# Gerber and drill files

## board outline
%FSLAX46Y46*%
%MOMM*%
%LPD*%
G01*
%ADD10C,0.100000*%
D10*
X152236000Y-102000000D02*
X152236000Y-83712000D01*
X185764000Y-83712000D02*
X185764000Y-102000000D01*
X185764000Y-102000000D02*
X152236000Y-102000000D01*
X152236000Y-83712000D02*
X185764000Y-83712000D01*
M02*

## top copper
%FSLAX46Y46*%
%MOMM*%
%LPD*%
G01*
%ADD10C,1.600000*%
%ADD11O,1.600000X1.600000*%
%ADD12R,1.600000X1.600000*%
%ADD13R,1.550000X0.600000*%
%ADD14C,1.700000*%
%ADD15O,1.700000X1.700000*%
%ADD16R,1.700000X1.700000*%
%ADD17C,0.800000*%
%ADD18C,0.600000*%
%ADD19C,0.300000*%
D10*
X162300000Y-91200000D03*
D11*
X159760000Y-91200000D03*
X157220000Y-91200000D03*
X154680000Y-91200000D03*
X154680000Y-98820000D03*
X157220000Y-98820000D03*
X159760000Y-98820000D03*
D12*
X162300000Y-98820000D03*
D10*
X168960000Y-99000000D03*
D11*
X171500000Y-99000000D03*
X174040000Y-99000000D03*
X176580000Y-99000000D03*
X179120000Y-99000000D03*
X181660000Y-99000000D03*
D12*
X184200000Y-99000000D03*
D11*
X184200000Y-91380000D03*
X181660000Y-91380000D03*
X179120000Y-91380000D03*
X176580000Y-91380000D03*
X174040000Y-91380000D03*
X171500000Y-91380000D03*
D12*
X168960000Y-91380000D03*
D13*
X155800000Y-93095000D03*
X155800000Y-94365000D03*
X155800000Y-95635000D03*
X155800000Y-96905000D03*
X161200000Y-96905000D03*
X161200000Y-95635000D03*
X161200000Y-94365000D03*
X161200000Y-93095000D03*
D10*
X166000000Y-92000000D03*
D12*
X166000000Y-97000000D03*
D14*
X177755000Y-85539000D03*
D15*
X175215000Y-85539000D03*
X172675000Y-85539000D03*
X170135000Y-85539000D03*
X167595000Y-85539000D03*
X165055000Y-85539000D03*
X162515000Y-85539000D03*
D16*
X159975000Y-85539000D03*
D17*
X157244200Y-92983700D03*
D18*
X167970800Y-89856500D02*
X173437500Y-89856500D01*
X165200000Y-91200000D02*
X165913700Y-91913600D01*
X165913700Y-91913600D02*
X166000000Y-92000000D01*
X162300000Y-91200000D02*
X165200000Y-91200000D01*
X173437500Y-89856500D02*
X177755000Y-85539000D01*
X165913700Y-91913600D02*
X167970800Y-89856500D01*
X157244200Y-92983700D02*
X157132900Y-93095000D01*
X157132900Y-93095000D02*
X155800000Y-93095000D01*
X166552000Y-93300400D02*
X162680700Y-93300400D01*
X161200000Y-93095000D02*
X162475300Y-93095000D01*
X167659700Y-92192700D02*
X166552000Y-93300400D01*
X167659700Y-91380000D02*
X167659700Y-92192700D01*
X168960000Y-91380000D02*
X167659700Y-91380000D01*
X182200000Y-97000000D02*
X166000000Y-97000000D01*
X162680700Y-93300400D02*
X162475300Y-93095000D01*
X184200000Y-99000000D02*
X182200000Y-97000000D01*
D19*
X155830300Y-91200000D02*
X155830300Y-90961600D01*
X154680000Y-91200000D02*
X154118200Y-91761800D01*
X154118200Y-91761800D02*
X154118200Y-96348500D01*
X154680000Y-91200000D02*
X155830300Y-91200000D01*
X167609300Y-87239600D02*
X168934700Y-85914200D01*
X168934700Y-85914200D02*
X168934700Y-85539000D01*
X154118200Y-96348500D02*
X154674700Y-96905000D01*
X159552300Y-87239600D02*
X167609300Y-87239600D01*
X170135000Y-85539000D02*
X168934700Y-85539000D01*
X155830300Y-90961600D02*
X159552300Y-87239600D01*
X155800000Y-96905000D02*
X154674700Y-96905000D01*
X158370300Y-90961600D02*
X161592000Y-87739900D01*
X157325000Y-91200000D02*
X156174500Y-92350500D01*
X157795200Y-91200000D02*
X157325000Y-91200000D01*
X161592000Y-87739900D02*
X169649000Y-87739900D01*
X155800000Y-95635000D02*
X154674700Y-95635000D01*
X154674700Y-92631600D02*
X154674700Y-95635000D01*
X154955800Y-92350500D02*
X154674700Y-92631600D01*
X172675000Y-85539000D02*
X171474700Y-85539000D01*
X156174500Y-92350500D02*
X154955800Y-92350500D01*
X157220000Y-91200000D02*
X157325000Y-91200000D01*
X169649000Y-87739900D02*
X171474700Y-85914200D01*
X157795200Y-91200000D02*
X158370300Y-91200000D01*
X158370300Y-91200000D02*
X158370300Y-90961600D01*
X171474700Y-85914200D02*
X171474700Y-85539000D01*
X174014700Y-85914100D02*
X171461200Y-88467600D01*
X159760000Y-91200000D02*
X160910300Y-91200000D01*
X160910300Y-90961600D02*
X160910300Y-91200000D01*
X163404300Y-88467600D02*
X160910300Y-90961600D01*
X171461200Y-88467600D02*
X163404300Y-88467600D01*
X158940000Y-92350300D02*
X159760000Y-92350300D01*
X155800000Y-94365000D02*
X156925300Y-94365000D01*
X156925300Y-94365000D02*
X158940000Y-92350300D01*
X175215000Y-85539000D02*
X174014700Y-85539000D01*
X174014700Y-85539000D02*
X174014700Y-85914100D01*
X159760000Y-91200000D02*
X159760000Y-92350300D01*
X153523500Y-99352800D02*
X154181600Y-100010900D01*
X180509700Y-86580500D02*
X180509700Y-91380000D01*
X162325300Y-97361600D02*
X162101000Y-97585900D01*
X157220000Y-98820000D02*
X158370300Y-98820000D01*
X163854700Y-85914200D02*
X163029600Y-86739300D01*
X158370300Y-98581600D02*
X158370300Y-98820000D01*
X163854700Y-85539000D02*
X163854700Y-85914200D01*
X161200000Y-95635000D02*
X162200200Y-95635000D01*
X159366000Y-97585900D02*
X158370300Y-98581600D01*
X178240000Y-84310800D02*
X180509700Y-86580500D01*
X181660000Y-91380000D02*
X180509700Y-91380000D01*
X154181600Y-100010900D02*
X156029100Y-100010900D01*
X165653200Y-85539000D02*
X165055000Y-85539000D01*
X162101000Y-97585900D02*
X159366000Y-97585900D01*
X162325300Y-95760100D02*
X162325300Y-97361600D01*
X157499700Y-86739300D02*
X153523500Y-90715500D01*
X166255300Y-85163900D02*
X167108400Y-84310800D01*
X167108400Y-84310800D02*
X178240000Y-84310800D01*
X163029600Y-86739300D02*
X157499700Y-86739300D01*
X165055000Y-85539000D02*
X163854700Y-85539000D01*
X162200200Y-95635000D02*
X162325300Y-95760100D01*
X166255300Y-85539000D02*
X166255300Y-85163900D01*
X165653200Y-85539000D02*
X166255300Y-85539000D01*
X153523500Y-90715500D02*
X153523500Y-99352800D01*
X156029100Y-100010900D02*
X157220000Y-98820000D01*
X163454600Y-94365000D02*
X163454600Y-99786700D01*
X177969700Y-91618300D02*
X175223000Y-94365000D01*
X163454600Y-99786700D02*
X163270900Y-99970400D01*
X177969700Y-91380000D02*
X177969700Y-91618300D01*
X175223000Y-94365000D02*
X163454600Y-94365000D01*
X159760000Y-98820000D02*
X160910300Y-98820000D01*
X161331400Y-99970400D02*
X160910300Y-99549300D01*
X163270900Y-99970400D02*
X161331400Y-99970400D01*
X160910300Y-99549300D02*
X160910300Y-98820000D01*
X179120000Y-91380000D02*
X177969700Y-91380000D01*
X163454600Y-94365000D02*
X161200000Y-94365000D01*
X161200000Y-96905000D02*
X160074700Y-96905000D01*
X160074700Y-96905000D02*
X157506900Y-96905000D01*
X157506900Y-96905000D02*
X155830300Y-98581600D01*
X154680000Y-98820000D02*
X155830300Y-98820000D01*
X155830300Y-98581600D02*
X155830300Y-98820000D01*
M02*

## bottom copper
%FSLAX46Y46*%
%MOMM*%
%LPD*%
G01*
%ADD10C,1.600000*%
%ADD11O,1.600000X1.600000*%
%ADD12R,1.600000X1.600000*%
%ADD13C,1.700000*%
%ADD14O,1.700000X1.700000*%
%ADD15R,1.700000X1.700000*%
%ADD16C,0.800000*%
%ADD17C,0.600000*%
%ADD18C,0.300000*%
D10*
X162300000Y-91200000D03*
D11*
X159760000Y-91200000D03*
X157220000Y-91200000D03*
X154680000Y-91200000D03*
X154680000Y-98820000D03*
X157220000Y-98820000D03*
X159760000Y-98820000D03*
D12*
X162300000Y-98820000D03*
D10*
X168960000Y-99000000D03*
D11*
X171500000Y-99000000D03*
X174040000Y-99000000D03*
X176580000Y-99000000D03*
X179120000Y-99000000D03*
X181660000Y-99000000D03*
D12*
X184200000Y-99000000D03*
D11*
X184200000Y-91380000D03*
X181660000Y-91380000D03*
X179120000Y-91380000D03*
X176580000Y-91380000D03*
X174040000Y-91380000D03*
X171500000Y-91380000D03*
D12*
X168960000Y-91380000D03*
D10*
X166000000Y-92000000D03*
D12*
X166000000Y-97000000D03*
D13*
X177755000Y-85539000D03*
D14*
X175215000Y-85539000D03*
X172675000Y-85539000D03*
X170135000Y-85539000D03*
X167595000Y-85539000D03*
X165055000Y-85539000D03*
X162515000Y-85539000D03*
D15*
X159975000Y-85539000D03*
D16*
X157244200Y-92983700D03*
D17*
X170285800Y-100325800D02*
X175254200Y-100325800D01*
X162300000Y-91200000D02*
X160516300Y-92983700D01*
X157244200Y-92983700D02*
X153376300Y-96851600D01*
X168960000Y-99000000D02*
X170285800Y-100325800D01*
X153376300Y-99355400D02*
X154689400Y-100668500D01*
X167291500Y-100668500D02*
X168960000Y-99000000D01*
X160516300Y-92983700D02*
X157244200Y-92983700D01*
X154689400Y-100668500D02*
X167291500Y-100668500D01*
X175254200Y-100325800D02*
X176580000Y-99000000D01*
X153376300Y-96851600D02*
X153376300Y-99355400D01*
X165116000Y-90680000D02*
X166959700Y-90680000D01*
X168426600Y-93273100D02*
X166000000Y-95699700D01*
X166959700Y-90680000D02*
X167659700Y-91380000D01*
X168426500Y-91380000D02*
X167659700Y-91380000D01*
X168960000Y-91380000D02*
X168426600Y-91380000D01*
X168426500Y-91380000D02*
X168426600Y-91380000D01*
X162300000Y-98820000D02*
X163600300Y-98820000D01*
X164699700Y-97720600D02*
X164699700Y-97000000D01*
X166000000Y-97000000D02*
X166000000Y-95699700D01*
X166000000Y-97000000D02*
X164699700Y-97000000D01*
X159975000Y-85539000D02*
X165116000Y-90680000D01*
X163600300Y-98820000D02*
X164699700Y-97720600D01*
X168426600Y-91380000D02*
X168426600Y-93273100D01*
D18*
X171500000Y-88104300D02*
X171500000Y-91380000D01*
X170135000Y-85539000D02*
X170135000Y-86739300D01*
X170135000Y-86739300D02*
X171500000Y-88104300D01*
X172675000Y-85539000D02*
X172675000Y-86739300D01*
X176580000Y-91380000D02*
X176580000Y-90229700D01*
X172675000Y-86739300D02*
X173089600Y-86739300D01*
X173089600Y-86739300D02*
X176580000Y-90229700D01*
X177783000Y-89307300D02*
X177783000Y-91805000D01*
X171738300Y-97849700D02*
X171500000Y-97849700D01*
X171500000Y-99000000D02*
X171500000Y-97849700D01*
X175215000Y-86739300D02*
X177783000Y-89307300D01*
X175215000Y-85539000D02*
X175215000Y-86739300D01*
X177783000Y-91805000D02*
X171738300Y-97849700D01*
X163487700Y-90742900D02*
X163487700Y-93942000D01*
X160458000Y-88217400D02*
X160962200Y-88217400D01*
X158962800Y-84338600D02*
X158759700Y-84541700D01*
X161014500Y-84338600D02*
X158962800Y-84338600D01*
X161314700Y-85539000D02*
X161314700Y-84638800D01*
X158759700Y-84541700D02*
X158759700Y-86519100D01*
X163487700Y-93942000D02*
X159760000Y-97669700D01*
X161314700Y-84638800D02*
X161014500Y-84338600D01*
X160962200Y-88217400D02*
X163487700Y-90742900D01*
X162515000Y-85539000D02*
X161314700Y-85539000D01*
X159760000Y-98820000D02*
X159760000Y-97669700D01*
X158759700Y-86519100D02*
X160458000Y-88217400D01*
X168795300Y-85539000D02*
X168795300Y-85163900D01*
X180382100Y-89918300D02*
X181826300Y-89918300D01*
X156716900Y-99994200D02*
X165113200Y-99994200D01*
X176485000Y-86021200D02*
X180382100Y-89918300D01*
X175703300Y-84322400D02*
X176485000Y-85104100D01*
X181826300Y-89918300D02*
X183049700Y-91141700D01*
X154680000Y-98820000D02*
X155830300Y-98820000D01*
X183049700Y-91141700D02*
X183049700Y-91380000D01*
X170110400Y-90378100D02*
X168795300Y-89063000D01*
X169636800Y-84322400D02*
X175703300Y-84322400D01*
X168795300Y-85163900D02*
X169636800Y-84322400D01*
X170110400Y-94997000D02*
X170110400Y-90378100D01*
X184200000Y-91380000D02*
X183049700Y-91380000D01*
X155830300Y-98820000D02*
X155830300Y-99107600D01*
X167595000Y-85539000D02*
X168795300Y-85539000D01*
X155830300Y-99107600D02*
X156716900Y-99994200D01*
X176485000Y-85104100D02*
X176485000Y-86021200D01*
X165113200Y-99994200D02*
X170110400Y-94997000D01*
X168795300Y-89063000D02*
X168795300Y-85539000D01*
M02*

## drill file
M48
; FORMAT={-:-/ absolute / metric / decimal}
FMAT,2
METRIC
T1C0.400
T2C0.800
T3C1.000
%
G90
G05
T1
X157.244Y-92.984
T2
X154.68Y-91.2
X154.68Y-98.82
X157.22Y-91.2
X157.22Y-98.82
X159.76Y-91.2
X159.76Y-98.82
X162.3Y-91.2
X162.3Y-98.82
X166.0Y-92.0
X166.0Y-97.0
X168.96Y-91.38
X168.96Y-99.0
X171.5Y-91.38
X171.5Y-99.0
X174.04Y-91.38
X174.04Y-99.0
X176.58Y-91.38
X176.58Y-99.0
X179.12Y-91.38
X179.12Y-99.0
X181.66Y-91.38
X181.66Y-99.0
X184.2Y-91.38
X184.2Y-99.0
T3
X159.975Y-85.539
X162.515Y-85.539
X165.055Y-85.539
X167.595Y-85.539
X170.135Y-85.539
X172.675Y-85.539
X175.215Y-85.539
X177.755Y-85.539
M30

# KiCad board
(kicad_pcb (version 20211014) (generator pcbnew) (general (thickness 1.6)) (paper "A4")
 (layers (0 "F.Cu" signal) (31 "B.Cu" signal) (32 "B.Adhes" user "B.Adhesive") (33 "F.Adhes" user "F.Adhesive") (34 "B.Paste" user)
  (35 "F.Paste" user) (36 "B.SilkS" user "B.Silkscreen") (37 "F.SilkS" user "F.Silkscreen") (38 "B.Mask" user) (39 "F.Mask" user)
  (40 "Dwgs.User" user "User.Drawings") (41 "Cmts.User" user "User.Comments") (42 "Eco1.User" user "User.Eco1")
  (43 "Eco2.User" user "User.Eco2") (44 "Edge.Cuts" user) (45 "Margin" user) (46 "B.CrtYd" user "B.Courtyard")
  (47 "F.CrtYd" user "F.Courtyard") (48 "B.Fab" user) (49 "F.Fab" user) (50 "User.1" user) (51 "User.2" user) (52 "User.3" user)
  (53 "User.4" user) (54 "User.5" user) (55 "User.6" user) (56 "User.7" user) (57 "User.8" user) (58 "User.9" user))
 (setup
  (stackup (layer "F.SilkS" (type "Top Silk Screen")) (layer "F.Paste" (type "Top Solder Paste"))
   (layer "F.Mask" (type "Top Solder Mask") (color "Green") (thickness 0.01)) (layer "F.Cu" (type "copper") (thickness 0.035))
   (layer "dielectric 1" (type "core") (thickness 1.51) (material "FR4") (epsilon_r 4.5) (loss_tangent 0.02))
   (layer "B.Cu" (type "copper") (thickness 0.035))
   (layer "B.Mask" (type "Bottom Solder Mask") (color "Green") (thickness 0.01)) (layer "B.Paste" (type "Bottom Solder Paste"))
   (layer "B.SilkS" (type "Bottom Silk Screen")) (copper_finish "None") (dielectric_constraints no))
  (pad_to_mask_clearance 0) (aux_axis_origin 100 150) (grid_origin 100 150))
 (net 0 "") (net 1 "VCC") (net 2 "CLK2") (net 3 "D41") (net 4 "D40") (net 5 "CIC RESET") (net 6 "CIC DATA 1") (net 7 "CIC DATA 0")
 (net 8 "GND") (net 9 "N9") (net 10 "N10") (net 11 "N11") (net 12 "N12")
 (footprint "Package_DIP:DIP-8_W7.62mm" (layer "F.Cu") (at 162.3 91.2 -90)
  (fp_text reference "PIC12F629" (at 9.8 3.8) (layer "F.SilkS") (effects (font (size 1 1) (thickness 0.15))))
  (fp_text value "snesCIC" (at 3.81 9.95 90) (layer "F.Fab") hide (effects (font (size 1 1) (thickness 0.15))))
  (pad "1" thru_hole circle (at 0 0 270) (size 1.6 1.6) (drill 0.8) (layers *.Cu *.Mask) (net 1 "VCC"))
  (pad "2" thru_hole oval (at 0 2.54 270) (size 1.6 1.6) (drill 0.8) (layers *.Cu *.Mask) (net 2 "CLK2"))
  (pad "3" thru_hole oval (at 0 5.08 270) (size 1.6 1.6) (drill 0.8) (layers *.Cu *.Mask) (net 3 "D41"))
  (pad "4" thru_hole oval (at 0 7.62 270) (size 1.6 1.6) (drill 0.8) (layers *.Cu *.Mask) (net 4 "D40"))
  (pad "5" thru_hole oval (at 7.62 7.62 270) (size 1.6 1.6) (drill 0.8) (layers *.Cu *.Mask) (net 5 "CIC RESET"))
  (pad "6" thru_hole oval (at 7.62 5.08 270) (size 1.6 1.6) (drill 0.8) (layers *.Cu *.Mask) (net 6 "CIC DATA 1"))
  (pad "7" thru_hole oval (at 7.62 2.54 270) (size 1.6 1.6) (drill 0.8) (layers *.Cu *.Mask) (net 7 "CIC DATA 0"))
  (pad "8" thru_hole rect (at 7.62 0 270) (size 1.6 1.6) (drill 0.8) (layers *.Cu *.Mask) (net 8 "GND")))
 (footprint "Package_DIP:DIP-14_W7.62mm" (layer "F.Cu") (at 168.96 99 90)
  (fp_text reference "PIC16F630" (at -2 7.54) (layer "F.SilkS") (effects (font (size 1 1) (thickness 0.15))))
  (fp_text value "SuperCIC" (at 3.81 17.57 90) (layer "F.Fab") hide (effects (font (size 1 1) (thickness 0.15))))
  (pad "1" thru_hole circle (at 0 0 90) (size 1.6 1.6) (drill 0.8) (layers *.Cu *.Mask) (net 1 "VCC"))
  (pad "2" thru_hole oval (at 0 2.54 90) (size 1.6 1.6) (drill 0.8) (layers *.Cu *.Mask) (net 2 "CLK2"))
  (pad "3" thru_hole oval (at 0 5.08 90) (size 1.6 1.6) (drill 0.8) (layers *.Cu *.Mask) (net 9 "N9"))
  (pad "4" thru_hole oval (at 0 7.62 90) (size 1.6 1.6) (drill 0.8) (layers *.Cu *.Mask) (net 1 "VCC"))
  (pad "5" thru_hole oval (at 0 10.16 90) (size 1.6 1.6) (drill 0.8) (layers *.Cu *.Mask) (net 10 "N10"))
  (pad "6" thru_hole oval (at 0 12.7 90) (size 1.6 1.6) (drill 0.8) (layers *.Cu *.Mask) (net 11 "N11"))
  (pad "7" thru_hole rect (at 0 15.24 90) (size 1.6 1.6) (drill 0.8) (layers *.Cu *.Mask) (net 8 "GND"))
  (pad "8" thru_hole oval (at 7.62 15.24 90) (size 1.6 1.6) (drill 0.8) (layers *.Cu *.Mask) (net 5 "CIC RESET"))
  (pad "9" thru_hole oval (at 7.62 12.7 90) (size 1.6 1.6) (drill 0.8) (layers *.Cu *.Mask) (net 6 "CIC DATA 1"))
  (pad "10" thru_hole oval (at 7.62 10.16 90) (size 1.6 1.6) (drill 0.8) (layers *.Cu *.Mask) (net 7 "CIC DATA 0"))
  (pad "11" thru_hole oval (at 7.62 7.62 90) (size 1.6 1.6) (drill 0.8) (layers *.Cu *.Mask) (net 3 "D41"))
  (pad "12" thru_hole oval (at 7.62 5.08 90) (size 1.6 1.6) (drill 0.8) (layers *.Cu *.Mask) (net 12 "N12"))
  (pad "13" thru_hole oval (at 7.62 2.54 90) (size 1.6 1.6) (drill 0.8) (layers *.Cu *.Mask) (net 4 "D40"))
  (pad "14" thru_hole rect (at 7.62 0 90) (size 1.6 1.6) (drill 0.8) (layers *.Cu *.Mask) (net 8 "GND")))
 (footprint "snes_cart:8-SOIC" (layer "F.Cu") (at 158.5 95 90)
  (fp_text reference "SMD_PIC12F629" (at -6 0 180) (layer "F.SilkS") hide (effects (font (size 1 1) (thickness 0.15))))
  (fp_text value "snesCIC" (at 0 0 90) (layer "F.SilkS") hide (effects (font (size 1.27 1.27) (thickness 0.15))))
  (pad "1" smd rect (at 1.905 -2.7 180) (size 1.55 0.6) (layers "F.Cu" "F.Paste" "F.Mask") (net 1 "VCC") (solder_mask_margin 0.1016))
  (pad "2" smd rect (at 0.635 -2.7 180) (size 1.55 0.6) (layers "F.Cu" "F.Paste" "F.Mask") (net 2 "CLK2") (solder_mask_margin 0.1016))
  (pad "3" smd rect (at -0.635 -2.7 180) (size 1.55 0.6) (layers "F.Cu" "F.Paste" "F.Mask") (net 3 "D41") (solder_mask_margin 0.1016))
  (pad "4" smd rect (at -1.905 -2.7 180) (size 1.55 0.6) (layers "F.Cu" "F.Paste" "F.Mask") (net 4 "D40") (solder_mask_margin 0.1016))
  (pad "5" smd rect (at -1.905 2.7 180) (size 1.55 0.6) (layers "F.Cu" "F.Paste" "F.Mask") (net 5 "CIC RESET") (solder_mask_margin 0.1016))
  (pad "6" smd rect (at -0.635 2.7 180) (size 1.55 0.6) (layers "F.Cu" "F.Paste" "F.Mask") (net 6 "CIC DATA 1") (solder_mask_margin 0.1016))
  (pad "7" smd rect (at 0.635 2.7 180) (size 1.55 0.6) (layers "F.Cu" "F.Paste" "F.Mask") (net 7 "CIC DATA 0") (solder_mask_margin 0.1016))
  (pad "8" smd rect (at 1.905 2.7 180) (size 1.55 0.6) (layers "F.Cu" "F.Paste" "F.Mask") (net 8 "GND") (solder_mask_margin 0.1016)))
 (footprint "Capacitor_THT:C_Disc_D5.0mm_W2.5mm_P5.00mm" (layer "F.Cu") (at 166 92 -90)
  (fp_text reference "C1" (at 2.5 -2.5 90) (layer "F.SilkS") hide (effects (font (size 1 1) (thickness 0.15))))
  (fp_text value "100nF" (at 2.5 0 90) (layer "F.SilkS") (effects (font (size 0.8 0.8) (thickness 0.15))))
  (pad "1" thru_hole circle (at 0 0 270) (size 1.6 1.6) (drill 0.8) (layers *.Cu *.Mask) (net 1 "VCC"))
  (pad "2" thru_hole rect (at 5 0 270) (size 1.6 1.6) (drill 0.8) (layers *.Cu *.Mask) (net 8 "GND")))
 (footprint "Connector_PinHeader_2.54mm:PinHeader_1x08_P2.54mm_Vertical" (layer "B.Cu") (at 177.755 85.539 90)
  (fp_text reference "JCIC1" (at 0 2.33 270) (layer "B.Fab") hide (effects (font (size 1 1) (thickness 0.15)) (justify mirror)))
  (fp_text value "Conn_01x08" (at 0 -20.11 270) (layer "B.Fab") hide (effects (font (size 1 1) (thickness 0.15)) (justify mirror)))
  (pad "1" thru_hole circle (at 0 0 90) (size 1.7 1.7) (drill 1) (layers *.Cu *.Mask) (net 1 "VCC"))
  (pad "2" thru_hole oval (at 0 -2.54 90) (size 1.7 1.7) (drill 1) (layers *.Cu *.Mask) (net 2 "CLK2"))
  (pad "3" thru_hole oval (at 0 -5.08 90) (size 1.7 1.7) (drill 1) (layers *.Cu *.Mask) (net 3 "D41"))
  (pad "4" thru_hole oval (at 0 -7.62 90) (size 1.7 1.7) (drill 1) (layers *.Cu *.Mask) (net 4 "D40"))
  (pad "5" thru_hole oval (at 0 -10.16 90) (size 1.7 1.7) (drill 1) (layers *.Cu *.Mask) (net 5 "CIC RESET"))
  (pad "6" thru_hole oval (at 0 -12.7 90) (size 1.7 1.7) (drill 1) (layers *.Cu *.Mask) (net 6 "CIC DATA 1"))
  (pad "7" thru_hole oval (at 0 -15.24 90) (size 1.7 1.7) (drill 1) (layers *.Cu *.Mask) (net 7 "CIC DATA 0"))
  (pad "8" thru_hole rect (at 0 -17.78 90) (size 1.7 1.7) (drill 1) (layers *.Cu *.Mask) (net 8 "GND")))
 (gr_line (start 152.236 102) (end 152.236 83.712) (layer "Edge.Cuts") (width 0.1))
 (gr_line (start 185.764 83.712) (end 185.764 102) (layer "Edge.Cuts") (width 0.1))
 (gr_line (start 185.764 102) (end 152.236 102) (layer "Edge.Cuts") (width 0.1))
 (gr_line (start 152.236 83.712) (end 185.764 83.712) (layer "Edge.Cuts") (width 0.1))
 (segment (start 167.9708 89.8565) (end 173.4375 89.8565) (width 0.6) (layer "F.Cu") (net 1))
 (segment (start 165.2 91.2) (end 165.9137 91.9136) (width 0.6) (layer "F.Cu") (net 1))
 (segment (start 165.9137 91.9136) (end 166 92) (width 0.6) (layer "F.Cu") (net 1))
 (segment (start 162.3 91.2) (end 165.2 91.2) (width 0.6) (layer "F.Cu") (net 1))
 (segment (start 173.4375 89.8565) (end 177.755 85.539) (width 0.6) (layer "F.Cu") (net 1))
 (segment (start 165.9137 91.9136) (end 167.9708 89.8565) (width 0.6) (layer "F.Cu") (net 1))
 (segment (start 157.2442 92.9837) (end 157.1329 93.095) (width 0.6) (layer "F.Cu") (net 1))
 (segment (start 157.1329 93.095) (end 155.8 93.095) (width 0.6) (layer "F.Cu") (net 1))
 (via (at 157.2442 92.9837) (size 0.8) (drill 0.4) (layers "F.Cu" "B.Cu") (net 1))
 (segment (start 170.2858 100.3258) (end 175.2542 100.3258) (width 0.6) (layer "B.Cu") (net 1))
 (segment (start 162.3 91.2) (end 160.5163 92.9837) (width 0.6) (layer "B.Cu") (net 1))
 (segment (start 157.2442 92.9837) (end 153.3763 96.8516) (width 0.6) (layer "B.Cu") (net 1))
 (segment (start 168.96 99) (end 170.2858 100.3258) (width 0.6) (layer "B.Cu") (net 1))
 (segment (start 153.3763 99.3554) (end 154.6894 100.6685) (width 0.6) (layer "B.Cu") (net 1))
 (segment (start 167.2915 100.6685) (end 168.96 99) (width 0.6) (layer "B.Cu") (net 1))
 (segment (start 160.5163 92.9837) (end 157.2442 92.9837) (width 0.6) (layer "B.Cu") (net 1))
 (segment (start 154.6894 100.6685) (end 167.2915 100.6685) (width 0.6) (layer "B.Cu") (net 1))
 (segment (start 175.2542 100.3258) (end 176.58 99) (width 0.6) (layer "B.Cu") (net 1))
 (segment (start 153.3763 96.8516) (end 153.3763 99.3554) (width 0.6) (layer "B.Cu") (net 1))
 (segment (start 166.552 93.3004) (end 162.6807 93.3004) (width 0.6) (layer "F.Cu") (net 8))
 (segment (start 161.2 93.095) (end 162.4753 93.095) (width 0.6) (layer "F.Cu") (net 8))
 (segment (start 167.6597 92.1927) (end 166.552 93.3004) (width 0.6) (layer "F.Cu") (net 8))
 (segment (start 167.6597 91.38) (end 167.6597 92.1927) (width 0.6) (layer "F.Cu") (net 8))
 (segment (start 168.96 91.38) (end 167.6597 91.38) (width 0.6) (layer "F.Cu") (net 8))
 (segment (start 182.2 97) (end 166 97) (width 0.6) (layer "F.Cu") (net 8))
 (segment (start 162.6807 93.3004) (end 162.4753 93.095) (width 0.6) (layer "F.Cu") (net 8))
 (segment (start 184.2 99) (end 182.2 97) (width 0.6) (layer "F.Cu") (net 8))
 (segment (start 165.116 90.68) (end 166.9597 90.68) (width 0.6) (layer "B.Cu") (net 8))
 (segment (start 168.4266 93.2731) (end 166 95.6997) (width 0.6) (layer "B.Cu") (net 8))
 (segment (start 166.9597 90.68) (end 167.6597 91.38) (width 0.6) (layer "B.Cu") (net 8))
 (segment (start 168.4265 91.38) (end 167.6597 91.38) (width 0.6) (layer "B.Cu") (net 8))
 (segment (start 168.96 91.38) (end 168.4266 91.38) (width 0.6) (layer "B.Cu") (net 8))
 (segment (start 168.4265 91.38) (end 168.4266 91.38) (width 0.6) (layer "B.Cu") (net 8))
 (segment (start 162.3 98.82) (end 163.6003 98.82) (width 0.6) (layer "B.Cu") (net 8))
 (segment (start 164.6997 97.7206) (end 164.6997 97) (width 0.6) (layer "B.Cu") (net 8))
 (segment (start 166 97) (end 166 95.6997) (width 0.6) (layer "B.Cu") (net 8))
 (segment (start 166 97) (end 164.6997 97) (width 0.6) (layer "B.Cu") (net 8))
 (segment (start 159.975 85.539) (end 165.116 90.68) (width 0.6) (layer "B.Cu") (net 8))
 (segment (start 163.6003 98.82) (end 164.6997 97.7206) (width 0.6) (layer "B.Cu") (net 8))
 (segment (start 168.4266 91.38) (end 168.4266 93.2731) (width 0.6) (layer "B.Cu") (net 8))
 (segment (start 155.8303 91.2) (end 155.8303 90.9616) (width 0.3) (layer "F.Cu") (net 4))
 (segment (start 154.68 91.2) (end 154.1182 91.7618) (width 0.3) (layer "F.Cu") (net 4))
 (segment (start 154.1182 91.7618) (end 154.1182 96.3485) (width 0.3) (layer "F.Cu") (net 4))
 (segment (start 154.68 91.2) (end 155.8303 91.2) (width 0.3) (layer "F.Cu") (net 4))
 (segment (start 167.6093 87.2396) (end 168.9347 85.9142) (width 0.3) (layer "F.Cu") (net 4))
 (segment (start 168.9347 85.9142) (end 168.9347 85.539) (width 0.3) (layer "F.Cu") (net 4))
 (segment (start 154.1182 96.3485) (end 154.6747 96.905) (width 0.3) (layer "F.Cu") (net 4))
 (segment (start 159.5523 87.2396) (end 167.6093 87.2396) (width 0.3) (layer "F.Cu") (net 4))
 (segment (start 170.135 85.539) (end 168.9347 85.539) (width 0.3) (layer "F.Cu") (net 4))
 (segment (start 155.8303 90.9616) (end 159.5523 87.2396) (width 0.3) (layer "F.Cu") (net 4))
 (segment (start 155.8 96.905) (end 154.6747 96.905) (width 0.3) (layer "F.Cu") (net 4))
 (segment (start 171.5 88.1043) (end 171.5 91.38) (width 0.3) (layer "B.Cu") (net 4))
 (segment (start 170.135 85.539) (end 170.135 86.7393) (width 0.3) (layer "B.Cu") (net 4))
 (segment (start 170.135 86.7393) (end 171.5 88.1043) (width 0.3) (layer "B.Cu") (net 4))
 (segment (start 158.3703 90.9616) (end 161.592 87.7399) (width 0.3) (layer "F.Cu") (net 3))
 (segment (start 157.325 91.2) (end 156.1745 92.3505) (width 0.3) (layer "F.Cu") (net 3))
 (segment (start 157.7952 91.2) (end 157.325 91.2) (width 0.3) (layer "F.Cu") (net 3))
 (segment (start 161.592 87.7399) (end 169.649 87.7399) (width 0.3) (layer "F.Cu") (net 3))
 (segment (start 155.8 95.635) (end 154.6747 95.635) (width 0.3) (layer "F.Cu") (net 3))
 (segment (start 154.6747 92.6316) (end 154.6747 95.635) (width 0.3) (layer "F.Cu") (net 3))
 (segment (start 154.9558 92.3505) (end 154.6747 92.6316) (width 0.3) (layer "F.Cu") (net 3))
 (segment (start 172.675 85.539) (end 171.4747 85.539) (width 0.3) (layer "F.Cu") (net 3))
 (segment (start 156.1745 92.3505) (end 154.9558 92.3505) (width 0.3) (layer "F.Cu") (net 3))
 (segment (start 157.22 91.2) (end 157.325 91.2) (width 0.3) (layer "F.Cu") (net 3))
 (segment (start 169.649 87.7399) (end 171.4747 85.9142) (width 0.3) (layer "F.Cu") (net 3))
 (segment (start 157.7952 91.2) (end 158.3703 91.2) (width 0.3) (layer "F.Cu") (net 3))
 (segment (start 158.3703 91.2) (end 158.3703 90.9616) (width 0.3) (layer "F.Cu") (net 3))
 (segment (start 171.4747 85.9142) (end 171.4747 85.539) (width 0.3) (layer "F.Cu") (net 3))
 (segment (start 172.675 85.539) (end 172.675 86.7393) (width 0.3) (layer "B.Cu") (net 3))
 (segment (start 176.58 91.38) (end 176.58 90.2297) (width 0.3) (layer "B.Cu") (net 3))
 (segment (start 172.675 86.7393) (end 173.0896 86.7393) (width 0.3) (layer "B.Cu") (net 3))
 (segment (start 173.0896 86.7393) (end 176.58 90.2297) (width 0.3) (layer "B.Cu") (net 3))
 (segment (start 174.0147 85.9141) (end 171.4612 88.4676) (width 0.3) (layer "F.Cu") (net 2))
 (segment (start 159.76 91.2) (end 160.9103 91.2) (width 0.3) (layer "F.Cu") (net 2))
 (segment (start 160.9103 90.9616) (end 160.9103 91.2) (width 0.3) (layer "F.Cu") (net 2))
 (segment (start 163.4043 88.4676) (end 160.9103 90.9616) (width 0.3) (layer "F.Cu") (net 2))
 (segment (start 171.4612 88.4676) (end 163.4043 88.4676) (width 0.3) (layer "F.Cu") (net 2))
 (segment (start 158.94 92.3503) (end 159.76 92.3503) (width 0.3) (layer "F.Cu") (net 2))
 (segment (start 155.8 94.365) (end 156.9253 94.365) (width 0.3) (layer "F.Cu") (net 2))
 (segment (start 156.9253 94.365) (end 158.94 92.3503) (width 0.3) (layer "F.Cu") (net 2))
 (segment (start 175.215 85.539) (end 174.0147 85.539) (width 0.3) (layer "F.Cu") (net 2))
 (segment (start 174.0147 85.539) (end 174.0147 85.9141) (width 0.3) (layer "F.Cu") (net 2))
 (segment (start 159.76 91.2) (end 159.76 92.3503) (width 0.3) (layer "F.Cu") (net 2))
 (segment (start 177.783 89.3073) (end 177.783 91.805) (width 0.3) (layer "B.Cu") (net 2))
 (segment (start 171.7383 97.8497) (end 171.5 97.8497) (width 0.3) (layer "B.Cu") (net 2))
 (segment (start 171.5 99) (end 171.5 97.8497) (width 0.3) (layer "B.Cu") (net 2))
 (segment (start 175.215 86.7393) (end 177.783 89.3073) (width 0.3) (layer "B.Cu") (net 2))
 (segment (start 175.215 85.539) (end 175.215 86.7393) (width 0.3) (layer "B.Cu") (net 2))
 (segment (start 177.783 91.805) (end 171.7383 97.8497) (width 0.3) (layer "B.Cu") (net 2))
 (segment (start 153.5235 99.3528) (end 154.1816 100.0109) (width 0.3) (layer "F.Cu") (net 6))
 (segment (start 180.5097 86.5805) (end 180.5097 91.38) (width 0.3) (layer "F.Cu") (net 6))
 (segment (start 162.3253 97.3616) (end 162.101 97.5859) (width 0.3) (layer "F.Cu") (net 6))
 (segment (start 157.22 98.82) (end 158.3703 98.82) (width 0.3) (layer "F.Cu") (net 6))
 (segment (start 163.8547 85.9142) (end 163.0296 86.7393) (width 0.3) (layer "F.Cu") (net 6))
 (segment (start 158.3703 98.5816) (end 158.3703 98.82) (width 0.3) (layer "F.Cu") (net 6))
 (segment (start 163.8547 85.539) (end 163.8547 85.9142) (width 0.3) (layer "F.Cu") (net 6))
 (segment (start 161.2 95.635) (end 162.2002 95.635) (width 0.3) (layer "F.Cu") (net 6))
 (segment (start 159.366 97.5859) (end 158.3703 98.5816) (width 0.3) (layer "F.Cu") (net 6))
 (segment (start 178.24 84.3108) (end 180.5097 86.5805) (width 0.3) (layer "F.Cu") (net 6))
 (segment (start 181.66 91.38) (end 180.5097 91.38) (width 0.3) (layer "F.Cu") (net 6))
 (segment (start 154.1816 100.0109) (end 156.0291 100.0109) (width 0.3) (layer "F.Cu") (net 6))
 (segment (start 165.6532 85.539) (end 165.055 85.539) (width 0.3) (layer "F.Cu") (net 6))
 (segment (start 162.101 97.5859) (end 159.366 97.5859) (width 0.3) (layer "F.Cu") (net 6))
 (segment (start 162.3253 95.7601) (end 162.3253 97.3616) (width 0.3) (layer "F.Cu") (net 6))
 (segment (start 157.4997 86.7393) (end 153.5235 90.7155) (width 0.3) (layer "F.Cu") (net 6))
 (segment (start 166.2553 85.1639) (end 167.1084 84.3108) (width 0.3) (layer "F.Cu") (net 6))
 (segment (start 167.1084 84.3108) (end 178.24 84.3108) (width 0.3) (layer "F.Cu") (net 6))
 (segment (start 163.0296 86.7393) (end 157.4997 86.7393) (width 0.3) (layer "F.Cu") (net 6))
 (segment (start 165.055 85.539) (end 163.8547 85.539) (width 0.3) (layer "F.Cu") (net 6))
 (segment (start 162.2002 95.635) (end 162.3253 95.7601) (width 0.3) (layer "F.Cu") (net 6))
 (segment (start 166.2553 85.539) (end 166.2553 85.1639) (width 0.3) (layer "F.Cu") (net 6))
 (segment (start 165.6532 85.539) (end 166.2553 85.539) (width 0.3) (layer "F.Cu") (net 6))
 (segment (start 153.5235 90.7155) (end 153.5235 99.3528) (width 0.3) (layer "F.Cu") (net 6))
 (segment (start 156.0291 100.0109) (end 157.22 98.82) (width 0.3) (layer "F.Cu") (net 6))
 (segment (start 163.4546 94.365) (end 163.4546 99.7867) (width 0.3) (layer "F.Cu") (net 7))
 (segment (start 177.9697 91.6183) (end 175.223 94.365) (width 0.3) (layer "F.Cu") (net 7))
 (segment (start 163.4546 99.7867) (end 163.2709 99.9704) (width 0.3) (layer "F.Cu") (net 7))
 (segment (start 177.9697 91.38) (end 177.9697 91.6183) (width 0.3) (layer "F.Cu") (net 7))
 (segment (start 175.223 94.365) (end 163.4546 94.365) (width 0.3) (layer "F.Cu") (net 7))
 (segment (start 159.76 98.82) (end 160.9103 98.82) (width 0.3) (layer "F.Cu") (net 7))
 (segment (start 161.3314 99.9704) (end 160.9103 99.5493) (width 0.3) (layer "F.Cu") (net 7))
 (segment (start 163.2709 99.9704) (end 161.3314 99.9704) (width 0.3) (layer "F.Cu") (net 7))
 (segment (start 160.9103 99.5493) (end 160.9103 98.82) (width 0.3) (layer "F.Cu") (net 7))
 (segment (start 179.12 91.38) (end 177.9697 91.38) (width 0.3) (layer "F.Cu") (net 7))
 (segment (start 163.4546 94.365) (end 161.2 94.365) (width 0.3) (layer "F.Cu") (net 7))
 (segment (start 163.4877 90.7429) (end 163.4877 93.942) (width 0.3) (layer "B.Cu") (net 7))
 (segment (start 160.458 88.2174) (end 160.9622 88.2174) (width 0.3) (layer "B.Cu") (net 7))
 (segment (start 158.9628 84.3386) (end 158.7597 84.5417) (width 0.3) (layer "B.Cu") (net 7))
 (segment (start 161.0145 84.3386) (end 158.9628 84.3386) (width 0.3) (layer "B.Cu") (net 7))
 (segment (start 161.3147 85.539) (end 161.3147 84.6388) (width 0.3) (layer "B.Cu") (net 7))
 (segment (start 158.7597 84.5417) (end 158.7597 86.5191) (width 0.3) (layer "B.Cu") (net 7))
 (segment (start 163.4877 93.942) (end 159.76 97.6697) (width 0.3) (layer "B.Cu") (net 7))
 (segment (start 161.3147 84.6388) (end 161.0145 84.3386) (width 0.3) (layer "B.Cu") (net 7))
 (segment (start 160.9622 88.2174) (end 163.4877 90.7429) (width 0.3) (layer "B.Cu") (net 7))
 (segment (start 162.515 85.539) (end 161.3147 85.539) (width 0.3) (layer "B.Cu") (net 7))
 (segment (start 159.76 98.82) (end 159.76 97.6697) (width 0.3) (layer "B.Cu") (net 7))
 (segment (start 158.7597 86.5191) (end 160.458 88.2174) (width 0.3) (layer "B.Cu") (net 7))
 (segment (start 161.2 96.905) (end 160.0747 96.905) (width 0.3) (layer "F.Cu") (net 5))
 (segment (start 160.0747 96.905) (end 157.5069 96.905) (width 0.3) (layer "F.Cu") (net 5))
 (segment (start 157.5069 96.905) (end 155.8303 98.5816) (width 0.3) (layer "F.Cu") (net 5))
 (segment (start 154.68 98.82) (end 155.8303 98.82) (width 0.3) (layer "F.Cu") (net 5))
 (segment (start 155.8303 98.5816) (end 155.8303 98.82) (width 0.3) (layer "F.Cu") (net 5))
 (segment (start 168.7953 85.539) (end 168.7953 85.1639) (width 0.3) (layer "B.Cu") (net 5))
 (segment (start 180.3821 89.9183) (end 181.8263 89.9183) (width 0.3) (layer "B.Cu") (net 5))
 (segment (start 156.7169 99.9942) (end 165.1132 99.9942) (width 0.3) (layer "B.Cu") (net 5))
 (segment (start 176.485 86.0212) (end 180.3821 89.9183) (width 0.3) (layer "B.Cu") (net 5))
 (segment (start 175.7033 84.3224) (end 176.485 85.1041) (width 0.3) (layer "B.Cu") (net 5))
 (segment (start 181.8263 89.9183) (end 183.0497 91.1417) (width 0.3) (layer "B.Cu") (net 5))
 (segment (start 154.68 98.82) (end 155.8303 98.82) (width 0.3) (layer "B.Cu") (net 5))
 (segment (start 183.0497 91.1417) (end 183.0497 91.38) (width 0.3) (layer "B.Cu") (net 5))
 (segment (start 170.1104 90.3781) (end 168.7953 89.063) (width 0.3) (layer "B.Cu") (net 5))
 (segment (start 169.6368 84.3224) (end 175.7033 84.3224) (width 0.3) (layer "B.Cu") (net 5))
 (segment (start 168.7953 85.1639) (end 169.6368 84.3224) (width 0.3) (layer "B.Cu") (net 5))
 (segment (start 170.1104 94.997) (end 170.1104 90.3781) (width 0.3) (layer "B.Cu") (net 5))
 (segment (start 184.2 91.38) (end 183.0497 91.38) (width 0.3) (layer "B.Cu") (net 5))
 (segment (start 155.8303 98.82) (end 155.8303 99.1076) (width 0.3) (layer "B.Cu") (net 5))
 (segment (start 167.595 85.539) (end 168.7953 85.539) (width 0.3) (layer "B.Cu") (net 5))
 (segment (start 155.8303 99.1076) (end 156.7169 99.9942) (width 0.3) (layer "B.Cu") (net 5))
 (segment (start 176.485 85.1041) (end 176.485 86.0212) (width 0.3) (layer "B.Cu") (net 5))
 (segment (start 165.1132 99.9942) (end 170.1104 94.997) (width 0.3) (layer "B.Cu") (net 5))
 (segment (start 168.7953 89.063) (end 168.7953 85.539) (width 0.3) (layer "B.Cu") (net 5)))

